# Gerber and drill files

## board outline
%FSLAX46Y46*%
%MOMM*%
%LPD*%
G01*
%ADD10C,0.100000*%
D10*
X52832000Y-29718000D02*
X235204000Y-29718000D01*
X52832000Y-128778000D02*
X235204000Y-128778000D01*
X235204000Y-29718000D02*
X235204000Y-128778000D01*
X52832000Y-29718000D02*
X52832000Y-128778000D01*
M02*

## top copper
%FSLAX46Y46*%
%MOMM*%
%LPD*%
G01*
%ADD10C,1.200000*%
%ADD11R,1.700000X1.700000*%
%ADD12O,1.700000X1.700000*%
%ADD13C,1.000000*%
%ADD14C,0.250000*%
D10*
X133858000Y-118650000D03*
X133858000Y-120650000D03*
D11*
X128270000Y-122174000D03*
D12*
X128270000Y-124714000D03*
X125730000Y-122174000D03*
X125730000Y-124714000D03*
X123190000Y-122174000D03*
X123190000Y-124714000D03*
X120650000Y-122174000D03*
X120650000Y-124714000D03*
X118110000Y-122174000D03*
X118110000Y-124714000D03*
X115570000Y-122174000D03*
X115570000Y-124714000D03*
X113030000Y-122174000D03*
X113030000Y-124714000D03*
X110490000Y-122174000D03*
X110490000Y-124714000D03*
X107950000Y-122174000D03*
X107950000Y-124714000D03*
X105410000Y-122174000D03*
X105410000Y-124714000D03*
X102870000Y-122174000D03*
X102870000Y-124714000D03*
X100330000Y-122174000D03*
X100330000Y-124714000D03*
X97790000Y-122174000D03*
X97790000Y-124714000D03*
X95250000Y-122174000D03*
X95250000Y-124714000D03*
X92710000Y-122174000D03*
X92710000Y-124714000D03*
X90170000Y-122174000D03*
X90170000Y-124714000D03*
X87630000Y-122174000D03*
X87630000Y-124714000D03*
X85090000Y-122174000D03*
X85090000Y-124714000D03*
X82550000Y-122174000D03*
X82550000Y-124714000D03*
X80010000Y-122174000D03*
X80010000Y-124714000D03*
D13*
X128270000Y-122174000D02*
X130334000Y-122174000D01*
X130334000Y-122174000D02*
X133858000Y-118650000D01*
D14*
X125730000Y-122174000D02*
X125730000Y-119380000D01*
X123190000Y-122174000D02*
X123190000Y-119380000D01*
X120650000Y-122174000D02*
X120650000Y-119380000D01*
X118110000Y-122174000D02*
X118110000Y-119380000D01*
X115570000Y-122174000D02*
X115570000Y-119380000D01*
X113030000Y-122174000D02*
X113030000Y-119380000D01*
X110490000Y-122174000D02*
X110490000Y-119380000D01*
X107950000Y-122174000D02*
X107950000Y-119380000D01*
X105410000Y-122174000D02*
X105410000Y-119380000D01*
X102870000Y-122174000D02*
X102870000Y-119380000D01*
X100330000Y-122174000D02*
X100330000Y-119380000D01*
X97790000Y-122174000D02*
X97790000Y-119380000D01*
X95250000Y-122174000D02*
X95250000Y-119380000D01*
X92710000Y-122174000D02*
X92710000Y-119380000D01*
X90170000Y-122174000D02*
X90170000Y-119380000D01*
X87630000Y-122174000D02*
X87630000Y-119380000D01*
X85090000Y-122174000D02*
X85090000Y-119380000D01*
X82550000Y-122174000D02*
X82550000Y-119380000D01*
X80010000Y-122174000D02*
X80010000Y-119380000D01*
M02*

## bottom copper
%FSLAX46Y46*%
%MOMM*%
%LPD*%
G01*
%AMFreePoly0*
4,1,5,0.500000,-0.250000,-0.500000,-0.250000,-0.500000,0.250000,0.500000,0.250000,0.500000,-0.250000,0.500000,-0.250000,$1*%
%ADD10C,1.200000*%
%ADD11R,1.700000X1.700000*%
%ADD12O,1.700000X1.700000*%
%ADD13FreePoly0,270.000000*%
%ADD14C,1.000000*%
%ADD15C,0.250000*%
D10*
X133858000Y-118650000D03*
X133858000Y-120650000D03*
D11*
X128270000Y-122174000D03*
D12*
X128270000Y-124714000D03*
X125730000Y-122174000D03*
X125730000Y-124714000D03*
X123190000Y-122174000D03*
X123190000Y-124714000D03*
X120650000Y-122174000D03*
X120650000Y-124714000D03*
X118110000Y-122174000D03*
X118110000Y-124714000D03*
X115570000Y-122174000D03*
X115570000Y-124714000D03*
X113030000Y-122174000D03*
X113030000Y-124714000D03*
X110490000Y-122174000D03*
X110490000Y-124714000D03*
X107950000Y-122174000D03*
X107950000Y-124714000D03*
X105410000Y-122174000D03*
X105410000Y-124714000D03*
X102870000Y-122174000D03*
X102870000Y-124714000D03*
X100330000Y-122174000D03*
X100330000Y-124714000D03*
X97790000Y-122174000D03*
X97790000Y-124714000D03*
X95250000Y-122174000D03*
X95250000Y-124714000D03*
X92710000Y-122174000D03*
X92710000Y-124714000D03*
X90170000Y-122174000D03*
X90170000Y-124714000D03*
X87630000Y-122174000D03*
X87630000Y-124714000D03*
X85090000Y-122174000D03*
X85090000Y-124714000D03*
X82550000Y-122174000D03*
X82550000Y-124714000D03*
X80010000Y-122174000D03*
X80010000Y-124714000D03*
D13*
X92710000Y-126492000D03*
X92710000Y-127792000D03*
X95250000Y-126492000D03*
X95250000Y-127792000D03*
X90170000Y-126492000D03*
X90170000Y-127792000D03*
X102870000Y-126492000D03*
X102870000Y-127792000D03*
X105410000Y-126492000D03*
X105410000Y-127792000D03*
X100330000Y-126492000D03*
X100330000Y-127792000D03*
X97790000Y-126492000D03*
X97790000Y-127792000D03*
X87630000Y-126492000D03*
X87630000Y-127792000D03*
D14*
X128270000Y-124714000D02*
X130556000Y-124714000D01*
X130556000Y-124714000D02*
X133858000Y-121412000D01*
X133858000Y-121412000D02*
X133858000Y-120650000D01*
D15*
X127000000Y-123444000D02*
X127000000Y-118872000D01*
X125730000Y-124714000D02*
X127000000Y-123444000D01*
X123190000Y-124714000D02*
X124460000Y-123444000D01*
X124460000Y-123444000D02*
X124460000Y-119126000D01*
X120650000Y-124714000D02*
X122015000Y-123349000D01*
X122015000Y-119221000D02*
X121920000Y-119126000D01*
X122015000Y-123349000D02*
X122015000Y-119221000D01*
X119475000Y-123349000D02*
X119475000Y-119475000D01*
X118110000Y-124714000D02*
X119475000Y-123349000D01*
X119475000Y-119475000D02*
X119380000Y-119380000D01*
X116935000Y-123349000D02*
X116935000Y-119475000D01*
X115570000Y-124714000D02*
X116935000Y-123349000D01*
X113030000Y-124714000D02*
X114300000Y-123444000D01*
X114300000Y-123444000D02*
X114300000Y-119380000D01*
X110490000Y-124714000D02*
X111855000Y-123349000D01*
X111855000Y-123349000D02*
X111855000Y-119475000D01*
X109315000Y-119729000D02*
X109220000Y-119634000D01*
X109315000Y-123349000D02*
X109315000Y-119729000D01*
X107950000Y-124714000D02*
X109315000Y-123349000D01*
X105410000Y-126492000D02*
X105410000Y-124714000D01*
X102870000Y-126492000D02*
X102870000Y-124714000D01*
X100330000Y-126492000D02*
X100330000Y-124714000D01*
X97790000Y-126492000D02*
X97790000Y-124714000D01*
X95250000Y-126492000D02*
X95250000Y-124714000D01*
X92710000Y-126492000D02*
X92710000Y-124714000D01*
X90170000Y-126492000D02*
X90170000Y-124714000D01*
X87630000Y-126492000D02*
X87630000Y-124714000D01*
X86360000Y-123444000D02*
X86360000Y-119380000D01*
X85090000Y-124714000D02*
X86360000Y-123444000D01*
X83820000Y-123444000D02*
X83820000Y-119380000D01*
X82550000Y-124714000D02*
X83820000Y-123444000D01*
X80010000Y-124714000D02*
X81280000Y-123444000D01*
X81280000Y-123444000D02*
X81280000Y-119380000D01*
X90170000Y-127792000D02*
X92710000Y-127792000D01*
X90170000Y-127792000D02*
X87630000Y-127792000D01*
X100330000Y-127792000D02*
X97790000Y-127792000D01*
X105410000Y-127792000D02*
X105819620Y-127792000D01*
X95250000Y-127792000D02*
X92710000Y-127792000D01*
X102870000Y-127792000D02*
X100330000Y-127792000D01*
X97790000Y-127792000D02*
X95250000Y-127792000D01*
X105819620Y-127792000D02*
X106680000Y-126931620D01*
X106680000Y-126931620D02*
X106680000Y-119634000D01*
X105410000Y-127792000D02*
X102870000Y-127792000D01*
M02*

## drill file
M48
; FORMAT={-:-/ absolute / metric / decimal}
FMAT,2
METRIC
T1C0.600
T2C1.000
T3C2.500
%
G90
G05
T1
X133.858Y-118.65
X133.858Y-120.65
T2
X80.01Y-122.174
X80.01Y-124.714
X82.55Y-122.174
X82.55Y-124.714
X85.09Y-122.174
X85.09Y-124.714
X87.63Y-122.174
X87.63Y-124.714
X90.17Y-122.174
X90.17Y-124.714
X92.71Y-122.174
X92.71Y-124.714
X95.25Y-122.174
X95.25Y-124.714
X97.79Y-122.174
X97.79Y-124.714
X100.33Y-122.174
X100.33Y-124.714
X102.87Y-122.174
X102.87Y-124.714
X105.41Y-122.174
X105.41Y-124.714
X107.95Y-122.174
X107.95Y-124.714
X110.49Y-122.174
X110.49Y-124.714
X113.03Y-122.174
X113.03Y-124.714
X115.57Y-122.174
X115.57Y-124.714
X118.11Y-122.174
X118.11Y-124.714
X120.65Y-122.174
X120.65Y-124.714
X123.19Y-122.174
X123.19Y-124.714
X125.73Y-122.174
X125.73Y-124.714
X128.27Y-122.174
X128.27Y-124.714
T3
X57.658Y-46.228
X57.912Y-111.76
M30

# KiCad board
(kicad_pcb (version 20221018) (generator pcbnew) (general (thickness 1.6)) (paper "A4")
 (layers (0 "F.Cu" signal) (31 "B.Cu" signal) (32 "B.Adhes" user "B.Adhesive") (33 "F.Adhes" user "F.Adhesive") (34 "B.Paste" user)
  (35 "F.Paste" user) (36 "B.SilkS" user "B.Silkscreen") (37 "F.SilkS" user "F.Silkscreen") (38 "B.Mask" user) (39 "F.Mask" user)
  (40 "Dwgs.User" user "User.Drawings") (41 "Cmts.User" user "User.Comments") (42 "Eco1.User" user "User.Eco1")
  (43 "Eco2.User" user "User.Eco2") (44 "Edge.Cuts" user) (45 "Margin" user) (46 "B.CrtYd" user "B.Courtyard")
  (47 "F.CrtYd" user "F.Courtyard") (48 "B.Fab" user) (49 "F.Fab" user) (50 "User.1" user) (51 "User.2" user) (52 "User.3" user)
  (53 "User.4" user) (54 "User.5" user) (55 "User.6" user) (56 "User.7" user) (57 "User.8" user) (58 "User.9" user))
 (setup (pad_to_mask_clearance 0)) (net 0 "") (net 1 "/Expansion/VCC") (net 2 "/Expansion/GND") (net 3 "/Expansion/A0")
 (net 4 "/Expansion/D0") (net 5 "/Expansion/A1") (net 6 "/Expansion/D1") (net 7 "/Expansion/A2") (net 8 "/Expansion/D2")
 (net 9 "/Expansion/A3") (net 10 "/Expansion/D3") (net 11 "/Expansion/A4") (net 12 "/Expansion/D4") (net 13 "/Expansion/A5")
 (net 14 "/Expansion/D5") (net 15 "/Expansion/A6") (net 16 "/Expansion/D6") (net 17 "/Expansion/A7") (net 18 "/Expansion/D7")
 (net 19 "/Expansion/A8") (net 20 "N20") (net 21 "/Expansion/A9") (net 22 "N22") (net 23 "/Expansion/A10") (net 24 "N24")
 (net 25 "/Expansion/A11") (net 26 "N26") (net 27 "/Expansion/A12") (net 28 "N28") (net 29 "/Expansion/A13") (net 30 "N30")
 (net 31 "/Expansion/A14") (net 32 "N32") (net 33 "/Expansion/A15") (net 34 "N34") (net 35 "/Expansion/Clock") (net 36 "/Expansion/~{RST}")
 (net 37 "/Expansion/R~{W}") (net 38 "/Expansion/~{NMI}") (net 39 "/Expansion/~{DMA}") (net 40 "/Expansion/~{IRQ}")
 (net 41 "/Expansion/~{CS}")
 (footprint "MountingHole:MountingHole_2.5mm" (layer "F.Cu") (at 57.912 111.76)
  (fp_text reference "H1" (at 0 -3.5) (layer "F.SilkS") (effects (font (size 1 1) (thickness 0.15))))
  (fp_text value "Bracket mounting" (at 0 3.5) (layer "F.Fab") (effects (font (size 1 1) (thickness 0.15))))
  (pad "" np_thru_hole circle (at 0 0) (size 2.5 2.5) (drill 2.5) (layers "*.Cu" "*.Mask")))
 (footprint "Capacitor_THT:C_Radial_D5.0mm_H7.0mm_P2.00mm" (layer "F.Cu") (at 133.858 118.65 -90)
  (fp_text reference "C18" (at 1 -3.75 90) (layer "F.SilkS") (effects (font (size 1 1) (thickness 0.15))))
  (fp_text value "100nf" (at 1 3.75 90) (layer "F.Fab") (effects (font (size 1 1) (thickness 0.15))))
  (pad "1" thru_hole circle (at 0 0 270) (size 1.2 1.2) (drill 0.6) (layers "*.Cu" "*.Mask") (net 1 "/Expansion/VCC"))
  (pad "2" thru_hole circle (at 2 0 270) (size 1.2 1.2) (drill 0.6) (layers "*.Cu" "*.Mask") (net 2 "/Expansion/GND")))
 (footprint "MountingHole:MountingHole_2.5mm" (layer "F.Cu") (at 57.658 46.228)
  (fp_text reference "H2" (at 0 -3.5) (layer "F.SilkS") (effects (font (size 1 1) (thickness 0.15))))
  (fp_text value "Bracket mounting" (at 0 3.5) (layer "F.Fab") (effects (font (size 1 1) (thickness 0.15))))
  (pad "" np_thru_hole circle (at 0 0) (size 2.5 2.5) (drill 2.5) (layers "*.Cu" "*.Mask")))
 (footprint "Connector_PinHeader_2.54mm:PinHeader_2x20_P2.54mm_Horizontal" (layer "F.Cu") (at 128.27 122.174 -90)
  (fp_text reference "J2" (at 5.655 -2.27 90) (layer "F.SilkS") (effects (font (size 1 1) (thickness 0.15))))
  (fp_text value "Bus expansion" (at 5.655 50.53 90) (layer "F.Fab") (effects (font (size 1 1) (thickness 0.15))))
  (pad "1" thru_hole rect (at 0 0 270) (size 1.7 1.7) (drill 1) (layers "*.Cu" "*.Mask") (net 1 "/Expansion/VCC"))
  (pad "2" thru_hole oval (at 2.54 0 270) (size 1.7 1.7) (drill 1) (layers "*.Cu" "*.Mask") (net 2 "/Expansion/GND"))
  (pad "3" thru_hole oval (at 0 2.54 270) (size 1.7 1.7) (drill 1) (layers "*.Cu" "*.Mask") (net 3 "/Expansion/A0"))
  (pad "4" thru_hole oval (at 2.54 2.54 270) (size 1.7 1.7) (drill 1) (layers "*.Cu" "*.Mask") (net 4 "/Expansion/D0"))
  (pad "5" thru_hole oval (at 0 5.08 270) (size 1.7 1.7) (drill 1) (layers "*.Cu" "*.Mask") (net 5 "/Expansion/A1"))
  (pad "6" thru_hole oval (at 2.54 5.08 270) (size 1.7 1.7) (drill 1) (layers "*.Cu" "*.Mask") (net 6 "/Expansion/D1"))
  (pad "7" thru_hole oval (at 0 7.62 270) (size 1.7 1.7) (drill 1) (layers "*.Cu" "*.Mask") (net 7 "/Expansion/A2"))
  (pad "8" thru_hole oval (at 2.54 7.62 270) (size 1.7 1.7) (drill 1) (layers "*.Cu" "*.Mask") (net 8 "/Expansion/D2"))
  (pad "9" thru_hole oval (at 0 10.16 270) (size 1.7 1.7) (drill 1) (layers "*.Cu" "*.Mask") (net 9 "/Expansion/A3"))
  (pad "10" thru_hole oval (at 2.54 10.16 270) (size 1.7 1.7) (drill 1) (layers "*.Cu" "*.Mask") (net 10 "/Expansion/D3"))
  (pad "11" thru_hole oval (at 0 12.7 270) (size 1.7 1.7) (drill 1) (layers "*.Cu" "*.Mask") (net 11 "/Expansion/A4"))
  (pad "12" thru_hole oval (at 2.54 12.7 270) (size 1.7 1.7) (drill 1) (layers "*.Cu" "*.Mask") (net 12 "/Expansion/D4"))
  (pad "13" thru_hole oval (at 0 15.24 270) (size 1.7 1.7) (drill 1) (layers "*.Cu" "*.Mask") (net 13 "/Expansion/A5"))
  (pad "14" thru_hole oval (at 2.54 15.24 270) (size 1.7 1.7) (drill 1) (layers "*.Cu" "*.Mask") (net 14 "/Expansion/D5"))
  (pad "15" thru_hole oval (at 0 17.78 270) (size 1.7 1.7) (drill 1) (layers "*.Cu" "*.Mask") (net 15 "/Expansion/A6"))
  (pad "16" thru_hole oval (at 2.54 17.78 270) (size 1.7 1.7) (drill 1) (layers "*.Cu" "*.Mask") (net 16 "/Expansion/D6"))
  (pad "17" thru_hole oval (at 0 20.32 270) (size 1.7 1.7) (drill 1) (layers "*.Cu" "*.Mask") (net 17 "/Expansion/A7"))
  (pad "18" thru_hole oval (at 2.54 20.32 270) (size 1.7 1.7) (drill 1) (layers "*.Cu" "*.Mask") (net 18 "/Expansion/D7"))
  (pad "19" thru_hole oval (at 0 22.86 270) (size 1.7 1.7) (drill 1) (layers "*.Cu" "*.Mask") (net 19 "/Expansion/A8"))
  (pad "20" thru_hole oval (at 2.54 22.86 270) (size 1.7 1.7) (drill 1) (layers "*.Cu" "*.Mask") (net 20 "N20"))
  (pad "21" thru_hole oval (at 0 25.4 270) (size 1.7 1.7) (drill 1) (layers "*.Cu" "*.Mask") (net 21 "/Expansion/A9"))
  (pad "22" thru_hole oval (at 2.54 25.4 270) (size 1.7 1.7) (drill 1) (layers "*.Cu" "*.Mask") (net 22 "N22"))
  (pad "23" thru_hole oval (at 0 27.94 270) (size 1.7 1.7) (drill 1) (layers "*.Cu" "*.Mask") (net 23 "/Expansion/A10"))
  (pad "24" thru_hole oval (at 2.54 27.94 270) (size 1.7 1.7) (drill 1) (layers "*.Cu" "*.Mask") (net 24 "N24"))
  (pad "25" thru_hole oval (at 0 30.48 270) (size 1.7 1.7) (drill 1) (layers "*.Cu" "*.Mask") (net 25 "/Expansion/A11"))
  (pad "26" thru_hole oval (at 2.54 30.48 270) (size 1.7 1.7) (drill 1) (layers "*.Cu" "*.Mask") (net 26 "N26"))
  (pad "27" thru_hole oval (at 0 33.02 270) (size 1.7 1.7) (drill 1) (layers "*.Cu" "*.Mask") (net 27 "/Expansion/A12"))
  (pad "28" thru_hole oval (at 2.54 33.02 270) (size 1.7 1.7) (drill 1) (layers "*.Cu" "*.Mask") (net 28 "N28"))
  (pad "29" thru_hole oval (at 0 35.56 270) (size 1.7 1.7) (drill 1) (layers "*.Cu" "*.Mask") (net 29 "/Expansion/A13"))
  (pad "30" thru_hole oval (at 2.54 35.56 270) (size 1.7 1.7) (drill 1) (layers "*.Cu" "*.Mask") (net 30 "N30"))
  (pad "31" thru_hole oval (at 0 38.1 270) (size 1.7 1.7) (drill 1) (layers "*.Cu" "*.Mask") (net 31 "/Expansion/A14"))
  (pad "32" thru_hole oval (at 2.54 38.1 270) (size 1.7 1.7) (drill 1) (layers "*.Cu" "*.Mask") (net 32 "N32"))
  (pad "33" thru_hole oval (at 0 40.64 270) (size 1.7 1.7) (drill 1) (layers "*.Cu" "*.Mask") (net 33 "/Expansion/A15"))
  (pad "34" thru_hole oval (at 2.54 40.64 270) (size 1.7 1.7) (drill 1) (layers "*.Cu" "*.Mask") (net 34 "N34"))
  (pad "35" thru_hole oval (at 0 43.18 270) (size 1.7 1.7) (drill 1) (layers "*.Cu" "*.Mask") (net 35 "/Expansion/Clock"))
  (pad "36" thru_hole oval (at 2.54 43.18 270) (size 1.7 1.7) (drill 1) (layers "*.Cu" "*.Mask") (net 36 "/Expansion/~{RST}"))
  (pad "37" thru_hole oval (at 0 45.72 270) (size 1.7 1.7) (drill 1) (layers "*.Cu" "*.Mask") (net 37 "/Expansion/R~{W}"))
  (pad "38" thru_hole oval (at 2.54 45.72 270) (size 1.7 1.7) (drill 1) (layers "*.Cu" "*.Mask") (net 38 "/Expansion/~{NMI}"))
  (pad "39" thru_hole oval (at 0 48.26 270) (size 1.7 1.7) (drill 1) (layers "*.Cu" "*.Mask") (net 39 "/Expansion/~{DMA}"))
  (pad "40" thru_hole oval (at 2.54 48.26 270) (size 1.7 1.7) (drill 1) (layers "*.Cu" "*.Mask") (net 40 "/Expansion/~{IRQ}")))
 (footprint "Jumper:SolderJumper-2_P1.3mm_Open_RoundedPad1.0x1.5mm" (layer "B.Cu") (at 92.71 127.142 -90)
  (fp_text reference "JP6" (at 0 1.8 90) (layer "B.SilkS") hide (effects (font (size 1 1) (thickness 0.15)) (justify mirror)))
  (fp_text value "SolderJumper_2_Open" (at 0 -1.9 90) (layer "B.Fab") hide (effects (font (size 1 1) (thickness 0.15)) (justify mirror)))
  (pad "1" smd custom (at -0.65 0 270) (size 1 0.5) (layers "B.Cu" "B.Mask") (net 30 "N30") (zone_connect 2) (thermal_bridge_angle 45)
   (options (clearance outline) (anchor rect)) (primitives))
  (pad "2" smd custom (at 0.65 0 270) (size 1 0.5) (layers "B.Cu" "B.Mask") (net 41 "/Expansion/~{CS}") (zone_connect 2)
   (thermal_bridge_angle 45) (options (clearance outline) (anchor rect)) (primitives)))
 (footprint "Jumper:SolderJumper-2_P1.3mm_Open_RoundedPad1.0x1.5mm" (layer "B.Cu") (at 95.25 127.142 -90)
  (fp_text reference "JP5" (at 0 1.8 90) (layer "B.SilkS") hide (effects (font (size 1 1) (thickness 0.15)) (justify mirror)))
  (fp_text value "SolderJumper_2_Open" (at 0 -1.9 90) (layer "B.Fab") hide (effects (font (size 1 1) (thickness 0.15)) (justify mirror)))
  (pad "1" smd custom (at -0.65 0 270) (size 1 0.5) (layers "B.Cu" "B.Mask") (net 28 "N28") (zone_connect 2) (thermal_bridge_angle 45)
   (options (clearance outline) (anchor rect)) (primitives))
  (pad "2" smd custom (at 0.65 0 270) (size 1 0.5) (layers "B.Cu" "B.Mask") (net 41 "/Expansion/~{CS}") (zone_connect 2)
   (thermal_bridge_angle 45) (options (clearance outline) (anchor rect)) (primitives)))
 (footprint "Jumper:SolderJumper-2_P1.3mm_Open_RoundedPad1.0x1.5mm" (layer "B.Cu") (at 90.17 127.142 -90)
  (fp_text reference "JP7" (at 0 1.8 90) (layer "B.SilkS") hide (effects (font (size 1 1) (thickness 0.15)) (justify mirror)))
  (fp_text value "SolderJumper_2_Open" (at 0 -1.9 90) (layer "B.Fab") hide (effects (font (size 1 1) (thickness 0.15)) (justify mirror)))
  (pad "1" smd custom (at -0.65 0 270) (size 1 0.5) (layers "B.Cu" "B.Mask") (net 32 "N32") (zone_connect 2) (thermal_bridge_angle 45)
   (options (clearance outline) (anchor rect)) (primitives))
  (pad "2" smd custom (at 0.65 0 270) (size 1 0.5) (layers "B.Cu" "B.Mask") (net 41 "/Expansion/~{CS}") (zone_connect 2)
   (thermal_bridge_angle 45) (options (clearance outline) (anchor rect)) (primitives)))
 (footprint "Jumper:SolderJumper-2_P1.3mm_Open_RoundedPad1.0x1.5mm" (layer "B.Cu") (at 102.87 127.142 -90)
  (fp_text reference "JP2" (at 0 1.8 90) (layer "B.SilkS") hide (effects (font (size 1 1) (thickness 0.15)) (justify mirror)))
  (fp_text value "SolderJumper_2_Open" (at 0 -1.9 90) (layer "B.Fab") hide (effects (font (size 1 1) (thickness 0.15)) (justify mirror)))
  (pad "1" smd custom (at -0.65 0 270) (size 1 0.5) (layers "B.Cu" "B.Mask") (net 22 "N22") (zone_connect 2) (thermal_bridge_angle 45)
   (options (clearance outline) (anchor rect)) (primitives))
  (pad "2" smd custom (at 0.65 0 270) (size 1 0.5) (layers "B.Cu" "B.Mask") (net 41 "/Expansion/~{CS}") (zone_connect 2)
   (thermal_bridge_angle 45) (options (clearance outline) (anchor rect)) (primitives)))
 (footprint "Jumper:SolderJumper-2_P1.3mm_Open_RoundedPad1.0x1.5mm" (layer "B.Cu") (at 105.41 127.142 -90)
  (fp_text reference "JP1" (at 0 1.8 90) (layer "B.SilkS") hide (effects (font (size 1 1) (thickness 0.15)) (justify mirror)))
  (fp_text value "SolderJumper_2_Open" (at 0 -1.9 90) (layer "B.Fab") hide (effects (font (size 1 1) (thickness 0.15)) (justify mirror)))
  (pad "1" smd custom (at -0.65 0 270) (size 1 0.5) (layers "B.Cu" "B.Mask") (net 20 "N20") (zone_connect 2) (thermal_bridge_angle 45)
   (options (clearance outline) (anchor rect)) (primitives))
  (pad "2" smd custom (at 0.65 0 270) (size 1 0.5) (layers "B.Cu" "B.Mask") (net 41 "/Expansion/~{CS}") (zone_connect 2)
   (thermal_bridge_angle 45) (options (clearance outline) (anchor rect)) (primitives)))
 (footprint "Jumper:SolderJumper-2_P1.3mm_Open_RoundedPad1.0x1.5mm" (layer "B.Cu") (at 100.33 127.142 -90)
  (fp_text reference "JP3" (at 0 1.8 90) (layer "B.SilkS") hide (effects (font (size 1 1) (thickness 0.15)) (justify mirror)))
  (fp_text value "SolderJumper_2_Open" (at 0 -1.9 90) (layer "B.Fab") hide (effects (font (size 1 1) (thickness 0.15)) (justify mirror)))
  (pad "1" smd custom (at -0.65 0 270) (size 1 0.5) (layers "B.Cu" "B.Mask") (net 24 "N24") (zone_connect 2) (thermal_bridge_angle 45)
   (options (clearance outline) (anchor rect)) (primitives))
  (pad "2" smd custom (at 0.65 0 270) (size 1 0.5) (layers "B.Cu" "B.Mask") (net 41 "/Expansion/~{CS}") (zone_connect 2)
   (thermal_bridge_angle 45) (options (clearance outline) (anchor rect)) (primitives)))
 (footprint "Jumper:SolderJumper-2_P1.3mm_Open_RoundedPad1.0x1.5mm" (layer "B.Cu") (at 97.79 127.142 -90)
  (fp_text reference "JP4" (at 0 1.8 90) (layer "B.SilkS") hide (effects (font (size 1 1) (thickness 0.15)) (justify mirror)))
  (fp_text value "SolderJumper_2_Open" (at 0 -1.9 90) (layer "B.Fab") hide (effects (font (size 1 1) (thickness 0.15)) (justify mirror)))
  (pad "1" smd custom (at -0.65 0 270) (size 1 0.5) (layers "B.Cu" "B.Mask") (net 26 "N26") (zone_connect 2) (thermal_bridge_angle 45)
   (options (clearance outline) (anchor rect)) (primitives))
  (pad "2" smd custom (at 0.65 0 270) (size 1 0.5) (layers "B.Cu" "B.Mask") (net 41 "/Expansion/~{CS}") (zone_connect 2)
   (thermal_bridge_angle 45) (options (clearance outline) (anchor rect)) (primitives)))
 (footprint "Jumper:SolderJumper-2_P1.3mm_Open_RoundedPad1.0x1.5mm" (layer "B.Cu") (at 87.63 127.142 -90)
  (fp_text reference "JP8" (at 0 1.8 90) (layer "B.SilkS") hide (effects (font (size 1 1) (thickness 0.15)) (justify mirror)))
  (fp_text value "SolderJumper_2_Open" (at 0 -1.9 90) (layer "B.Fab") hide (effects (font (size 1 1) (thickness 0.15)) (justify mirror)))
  (pad "1" smd custom (at -0.65 0 270) (size 1 0.5) (layers "B.Cu" "B.Mask") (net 34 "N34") (zone_connect 2) (thermal_bridge_angle 45)
   (options (clearance outline) (anchor rect)) (primitives))
  (pad "2" smd custom (at 0.65 0 270) (size 1 0.5) (layers "B.Cu" "B.Mask") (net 41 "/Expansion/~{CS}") (zone_connect 2)
   (thermal_bridge_angle 45) (options (clearance outline) (anchor rect)) (primitives)))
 (gr_line (start 52.832 29.718) (end 235.204 29.718) (stroke (width 0.1) (type default)) (layer "Edge.Cuts"))
 (gr_line (start 52.832 128.778) (end 235.204 128.778) (stroke (width 0.1) (type default)) (layer "Edge.Cuts"))
 (gr_line (start 235.204 29.718) (end 235.204 128.778) (stroke (width 0.1) (type default)) (layer "Edge.Cuts"))
 (gr_line (start 52.832 29.718) (end 52.832 128.778) (stroke (width 0.1) (type default)) (layer "Edge.Cuts"))
 (segment (start 128.27 122.174) (end 130.334 122.174) (width 1) (layer "F.Cu") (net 1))
 (segment (start 130.334 122.174) (end 133.858 118.65) (width 1) (layer "F.Cu") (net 1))
 (segment (start 128.27 124.714) (end 130.556 124.714) (width 1) (layer "B.Cu") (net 2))
 (segment (start 130.556 124.714) (end 133.858 121.412) (width 1) (layer "B.Cu") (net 2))
 (segment (start 133.858 121.412) (end 133.858 120.65) (width 1) (layer "B.Cu") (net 2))
 (segment (start 125.73 122.174) (end 125.73 119.38) (width 0.25) (layer "F.Cu") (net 3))
 (segment (start 127 123.444) (end 127 118.872) (width 0.25) (layer "B.Cu") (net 4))
 (segment (start 125.73 124.714) (end 127 123.444) (width 0.25) (layer "B.Cu") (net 4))
 (segment (start 123.19 122.174) (end 123.19 119.38) (width 0.25) (layer "F.Cu") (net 5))
 (segment (start 123.19 124.714) (end 124.46 123.444) (width 0.25) (layer "B.Cu") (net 6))
 (segment (start 124.46 123.444) (end 124.46 119.126) (width 0.25) (layer "B.Cu") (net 6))
 (segment (start 120.65 122.174) (end 120.65 119.38) (width 0.25) (layer "F.Cu") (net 7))
 (segment (start 120.65 124.714) (end 122.015 123.349) (width 0.25) (layer "B.Cu") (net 8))
 (segment (start 122.015 119.221) (end 121.92 119.126) (width 0.25) (layer "B.Cu") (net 8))
 (segment (start 122.015 123.349) (end 122.015 119.221) (width 0.25) (layer "B.Cu") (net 8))
 (segment (start 118.11 122.174) (end 118.11 119.38) (width 0.25) (layer "F.Cu") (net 9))
 (segment (start 119.475 123.349) (end 119.475 119.475) (width 0.25) (layer "B.Cu") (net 10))
 (segment (start 118.11 124.714) (end 119.475 123.349) (width 0.25) (layer "B.Cu") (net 10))
 (segment (start 119.475 119.475) (end 119.38 119.38) (width 0.25) (layer "B.Cu") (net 10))
 (segment (start 115.57 122.174) (end 115.57 119.38) (width 0.25) (layer "F.Cu") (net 11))
 (segment (start 116.935 123.349) (end 116.935 119.475) (width 0.25) (layer "B.Cu") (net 12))
 (segment (start 115.57 124.714) (end 116.935 123.349) (width 0.25) (layer "B.Cu") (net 12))
 (segment (start 113.03 122.174) (end 113.03 119.38) (width 0.25) (layer "F.Cu") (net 13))
 (segment (start 113.03 124.714) (end 114.3 123.444) (width 0.25) (layer "B.Cu") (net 14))
 (segment (start 114.3 123.444) (end 114.3 119.38) (width 0.25) (layer "B.Cu") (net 14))
 (segment (start 110.49 122.174) (end 110.49 119.38) (width 0.25) (layer "F.Cu") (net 15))
 (segment (start 110.49 124.714) (end 111.855 123.349) (width 0.25) (layer "B.Cu") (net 16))
 (segment (start 111.855 123.349) (end 111.855 119.475) (width 0.25) (layer "B.Cu") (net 16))
 (segment (start 107.95 122.174) (end 107.95 119.38) (width 0.25) (layer "F.Cu") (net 17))
 (segment (start 109.315 119.729) (end 109.22 119.634) (width 0.25) (layer "B.Cu") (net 18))
 (segment (start 109.315 123.349) (end 109.315 119.729) (width 0.25) (layer "B.Cu") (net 18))
 (segment (start 107.95 124.714) (end 109.315 123.349) (width 0.25) (layer "B.Cu") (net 18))
 (segment (start 105.41 122.174) (end 105.41 119.38) (width 0.25) (layer "F.Cu") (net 19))
 (segment (start 105.41 126.492) (end 105.41 124.714) (width 0.25) (layer "B.Cu") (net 20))
 (segment (start 102.87 122.174) (end 102.87 119.38) (width 0.25) (layer "F.Cu") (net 21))
 (segment (start 102.87 126.492) (end 102.87 124.714) (width 0.25) (layer "B.Cu") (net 22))
 (segment (start 100.33 122.174) (end 100.33 119.38) (width 0.25) (layer "F.Cu") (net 23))
 (segment (start 100.33 126.492) (end 100.33 124.714) (width 0.25) (layer "B.Cu") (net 24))
 (segment (start 97.79 122.174) (end 97.79 119.38) (width 0.25) (layer "F.Cu") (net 25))
 (segment (start 97.79 126.492) (end 97.79 124.714) (width 0.25) (layer "B.Cu") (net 26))
 (segment (start 95.25 122.174) (end 95.25 119.38) (width 0.25) (layer "F.Cu") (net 27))
 (segment (start 95.25 126.492) (end 95.25 124.714) (width 0.25) (layer "B.Cu") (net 28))
 (segment (start 92.71 122.174) (end 92.71 119.38) (width 0.25) (layer "F.Cu") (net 29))
 (segment (start 92.71 126.492) (end 92.71 124.714) (width 0.25) (layer "B.Cu") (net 30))
 (segment (start 90.17 122.174) (end 90.17 119.38) (width 0.25) (layer "F.Cu") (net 31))
 (segment (start 90.17 126.492) (end 90.17 124.714) (width 0.25) (layer "B.Cu") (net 32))
 (segment (start 87.63 122.174) (end 87.63 119.38) (width 0.25) (layer "F.Cu") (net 33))
 (segment (start 87.63 126.492) (end 87.63 124.714) (width 0.25) (layer "B.Cu") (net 34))
 (segment (start 85.09 122.174) (end 85.09 119.38) (width 0.25) (layer "F.Cu") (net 35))
 (segment (start 86.36 123.444) (end 86.36 119.38) (width 0.25) (layer "B.Cu") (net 36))
 (segment (start 85.09 124.714) (end 86.36 123.444) (width 0.25) (layer "B.Cu") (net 36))
 (segment (start 82.55 122.174) (end 82.55 119.38) (width 0.25) (layer "F.Cu") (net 37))
 (segment (start 83.82 123.444) (end 83.82 119.38) (width 0.25) (layer "B.Cu") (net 38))
 (segment (start 82.55 124.714) (end 83.82 123.444) (width 0.25) (layer "B.Cu") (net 38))
 (segment (start 80.01 122.174) (end 80.01 119.38) (width 0.25) (layer "F.Cu") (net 39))
 (segment (start 80.01 124.714) (end 81.28 123.444) (width 0.25) (layer "B.Cu") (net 40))
 (segment (start 81.28 123.444) (end 81.28 119.38) (width 0.25) (layer "B.Cu") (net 40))
 (segment (start 90.17 127.792) (end 92.71 127.792) (width 0.25) (layer "B.Cu") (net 41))
 (segment (start 90.17 127.792) (end 87.63 127.792) (width 0.25) (layer "B.Cu") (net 41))
 (segment (start 100.33 127.792) (end 97.79 127.792) (width 0.25) (layer "B.Cu") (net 41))
 (segment (start 105.41 127.792) (end 105.81962 127.792) (width 0.25) (layer "B.Cu") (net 41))
 (segment (start 95.25 127.792) (end 92.71 127.792) (width 0.25) (layer "B.Cu") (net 41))
 (segment (start 102.87 127.792) (end 100.33 127.792) (width 0.25) (layer "B.Cu") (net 41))
 (segment (start 97.79 127.792) (end 95.25 127.792) (width 0.25) (layer "B.Cu") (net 41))
 (segment (start 105.81962 127.792) (end 106.68 126.93162) (width 0.25) (layer "B.Cu") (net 41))
 (segment (start 106.68 126.93162) (end 106.68 119.634) (width 0.25) (layer "B.Cu") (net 41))
 (segment (start 105.41 127.792) (end 102.87 127.792) (width 0.25) (layer "B.Cu") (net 41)))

